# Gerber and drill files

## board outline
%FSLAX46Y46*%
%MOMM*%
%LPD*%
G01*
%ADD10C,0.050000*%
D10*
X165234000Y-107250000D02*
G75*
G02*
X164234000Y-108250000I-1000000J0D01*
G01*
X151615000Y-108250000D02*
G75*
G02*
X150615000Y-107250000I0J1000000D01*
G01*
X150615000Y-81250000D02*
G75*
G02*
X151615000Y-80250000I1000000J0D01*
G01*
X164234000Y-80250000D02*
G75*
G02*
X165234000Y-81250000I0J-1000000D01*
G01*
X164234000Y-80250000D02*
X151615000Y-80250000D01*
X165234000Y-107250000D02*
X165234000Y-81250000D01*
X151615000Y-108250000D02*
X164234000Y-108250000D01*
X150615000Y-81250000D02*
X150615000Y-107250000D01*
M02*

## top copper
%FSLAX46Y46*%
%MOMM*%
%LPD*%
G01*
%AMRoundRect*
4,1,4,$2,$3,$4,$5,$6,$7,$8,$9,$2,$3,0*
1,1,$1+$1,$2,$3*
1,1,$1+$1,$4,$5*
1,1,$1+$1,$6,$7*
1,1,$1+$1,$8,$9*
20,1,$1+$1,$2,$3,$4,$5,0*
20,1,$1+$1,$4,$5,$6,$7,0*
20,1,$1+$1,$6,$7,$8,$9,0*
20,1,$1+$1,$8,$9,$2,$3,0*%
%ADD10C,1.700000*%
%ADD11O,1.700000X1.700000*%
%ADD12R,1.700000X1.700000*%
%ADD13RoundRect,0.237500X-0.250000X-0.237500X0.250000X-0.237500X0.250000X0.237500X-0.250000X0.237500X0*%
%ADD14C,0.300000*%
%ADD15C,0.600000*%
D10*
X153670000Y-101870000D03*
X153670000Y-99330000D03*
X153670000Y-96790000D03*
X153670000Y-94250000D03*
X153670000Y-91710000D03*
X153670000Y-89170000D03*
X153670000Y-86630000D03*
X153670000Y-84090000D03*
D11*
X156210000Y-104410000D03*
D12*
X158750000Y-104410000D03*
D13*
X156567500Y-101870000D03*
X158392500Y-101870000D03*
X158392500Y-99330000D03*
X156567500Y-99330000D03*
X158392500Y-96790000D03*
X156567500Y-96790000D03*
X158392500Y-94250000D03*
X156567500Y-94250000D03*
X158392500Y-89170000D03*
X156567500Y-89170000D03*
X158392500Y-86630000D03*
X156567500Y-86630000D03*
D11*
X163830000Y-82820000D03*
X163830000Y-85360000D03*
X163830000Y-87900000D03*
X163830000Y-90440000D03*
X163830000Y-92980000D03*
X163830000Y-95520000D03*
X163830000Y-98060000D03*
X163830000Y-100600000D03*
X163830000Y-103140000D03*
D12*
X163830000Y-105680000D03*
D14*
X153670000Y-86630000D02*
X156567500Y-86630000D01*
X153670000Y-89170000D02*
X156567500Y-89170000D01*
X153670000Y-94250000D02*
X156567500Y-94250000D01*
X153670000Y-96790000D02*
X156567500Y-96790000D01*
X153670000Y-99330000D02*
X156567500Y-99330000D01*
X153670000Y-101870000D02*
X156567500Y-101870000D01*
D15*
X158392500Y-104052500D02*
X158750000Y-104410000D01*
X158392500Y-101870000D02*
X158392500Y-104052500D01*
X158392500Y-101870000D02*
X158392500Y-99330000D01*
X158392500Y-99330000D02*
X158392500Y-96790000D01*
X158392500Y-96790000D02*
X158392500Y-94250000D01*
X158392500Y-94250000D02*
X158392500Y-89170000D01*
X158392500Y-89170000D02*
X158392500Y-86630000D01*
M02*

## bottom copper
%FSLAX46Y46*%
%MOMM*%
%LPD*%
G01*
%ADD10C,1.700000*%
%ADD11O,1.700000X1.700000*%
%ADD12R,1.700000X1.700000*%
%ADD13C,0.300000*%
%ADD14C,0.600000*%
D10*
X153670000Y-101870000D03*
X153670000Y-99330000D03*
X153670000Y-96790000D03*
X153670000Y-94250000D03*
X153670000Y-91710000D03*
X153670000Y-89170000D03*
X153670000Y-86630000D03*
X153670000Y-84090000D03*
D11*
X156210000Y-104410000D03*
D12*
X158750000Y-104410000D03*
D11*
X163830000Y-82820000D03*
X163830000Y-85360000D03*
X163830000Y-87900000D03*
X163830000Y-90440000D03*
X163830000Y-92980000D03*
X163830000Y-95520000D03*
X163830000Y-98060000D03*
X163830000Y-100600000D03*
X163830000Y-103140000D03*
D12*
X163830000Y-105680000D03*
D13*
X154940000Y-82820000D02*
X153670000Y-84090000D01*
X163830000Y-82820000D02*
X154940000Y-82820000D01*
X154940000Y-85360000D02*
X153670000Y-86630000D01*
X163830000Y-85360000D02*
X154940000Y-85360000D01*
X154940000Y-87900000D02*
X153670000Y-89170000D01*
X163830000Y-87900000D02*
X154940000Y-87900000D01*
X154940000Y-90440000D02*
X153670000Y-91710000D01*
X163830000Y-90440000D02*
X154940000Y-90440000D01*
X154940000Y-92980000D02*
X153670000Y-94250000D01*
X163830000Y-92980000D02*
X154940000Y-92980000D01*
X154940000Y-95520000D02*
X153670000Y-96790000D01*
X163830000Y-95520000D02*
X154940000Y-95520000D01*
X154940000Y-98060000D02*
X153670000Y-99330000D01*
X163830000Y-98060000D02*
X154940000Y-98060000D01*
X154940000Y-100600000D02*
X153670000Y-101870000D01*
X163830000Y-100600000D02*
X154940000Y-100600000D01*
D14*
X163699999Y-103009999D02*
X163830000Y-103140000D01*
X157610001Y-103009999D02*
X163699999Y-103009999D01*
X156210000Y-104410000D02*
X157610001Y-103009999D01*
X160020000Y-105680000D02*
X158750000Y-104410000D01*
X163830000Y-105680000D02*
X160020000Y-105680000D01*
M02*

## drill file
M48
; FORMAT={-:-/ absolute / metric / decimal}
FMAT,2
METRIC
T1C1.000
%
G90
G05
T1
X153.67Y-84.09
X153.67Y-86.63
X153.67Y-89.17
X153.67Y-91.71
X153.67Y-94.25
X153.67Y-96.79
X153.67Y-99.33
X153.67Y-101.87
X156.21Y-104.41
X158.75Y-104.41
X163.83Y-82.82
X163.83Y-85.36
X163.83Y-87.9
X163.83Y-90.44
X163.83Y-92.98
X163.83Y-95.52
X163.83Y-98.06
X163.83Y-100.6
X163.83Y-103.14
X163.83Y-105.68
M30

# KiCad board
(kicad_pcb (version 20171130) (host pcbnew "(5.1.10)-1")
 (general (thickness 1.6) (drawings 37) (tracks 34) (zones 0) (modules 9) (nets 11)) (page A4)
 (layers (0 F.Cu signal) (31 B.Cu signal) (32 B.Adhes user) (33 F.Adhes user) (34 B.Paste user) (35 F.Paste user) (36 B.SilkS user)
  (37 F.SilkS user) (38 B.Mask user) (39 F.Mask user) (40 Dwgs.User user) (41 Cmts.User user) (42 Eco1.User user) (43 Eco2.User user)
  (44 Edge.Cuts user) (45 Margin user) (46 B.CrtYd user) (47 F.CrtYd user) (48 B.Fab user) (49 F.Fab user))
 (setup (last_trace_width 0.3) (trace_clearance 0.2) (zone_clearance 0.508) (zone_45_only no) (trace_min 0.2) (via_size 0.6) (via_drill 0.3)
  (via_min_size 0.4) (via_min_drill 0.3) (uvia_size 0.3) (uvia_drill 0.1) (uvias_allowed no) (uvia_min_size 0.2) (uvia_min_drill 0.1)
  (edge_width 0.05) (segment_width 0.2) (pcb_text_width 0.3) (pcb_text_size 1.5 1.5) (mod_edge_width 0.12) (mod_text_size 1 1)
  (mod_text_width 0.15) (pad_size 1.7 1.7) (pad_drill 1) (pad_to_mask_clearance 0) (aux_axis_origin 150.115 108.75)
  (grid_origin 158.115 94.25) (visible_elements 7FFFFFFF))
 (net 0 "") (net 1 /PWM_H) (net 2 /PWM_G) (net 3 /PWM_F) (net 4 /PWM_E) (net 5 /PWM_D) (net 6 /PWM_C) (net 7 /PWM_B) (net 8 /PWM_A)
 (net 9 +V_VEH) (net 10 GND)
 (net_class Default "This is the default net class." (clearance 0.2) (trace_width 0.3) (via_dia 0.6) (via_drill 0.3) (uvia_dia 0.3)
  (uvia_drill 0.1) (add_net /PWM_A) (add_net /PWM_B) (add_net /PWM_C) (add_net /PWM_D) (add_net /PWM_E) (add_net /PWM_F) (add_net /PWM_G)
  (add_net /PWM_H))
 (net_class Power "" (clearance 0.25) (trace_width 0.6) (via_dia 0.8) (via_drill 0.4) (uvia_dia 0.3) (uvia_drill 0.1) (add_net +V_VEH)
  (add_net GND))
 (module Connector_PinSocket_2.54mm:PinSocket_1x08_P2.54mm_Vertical (layer B.Cu) (at 153.67 84.09 180)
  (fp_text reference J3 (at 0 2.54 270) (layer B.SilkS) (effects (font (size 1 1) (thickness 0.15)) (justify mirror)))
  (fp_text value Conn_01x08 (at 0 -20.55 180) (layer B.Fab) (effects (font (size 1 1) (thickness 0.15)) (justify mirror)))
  (pad 8 thru_hole circle (at 0 -17.78 180) (size 1.7 1.7) (drill 1) (layers *.Cu *.Mask) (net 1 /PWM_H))
  (pad 7 thru_hole circle (at 0 -15.24 180) (size 1.7 1.7) (drill 1) (layers *.Cu *.Mask) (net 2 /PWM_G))
  (pad 6 thru_hole circle (at 0 -12.7 180) (size 1.7 1.7) (drill 1) (layers *.Cu *.Mask) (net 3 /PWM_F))
  (pad 5 thru_hole circle (at 0 -10.16 180) (size 1.7 1.7) (drill 1) (layers *.Cu *.Mask) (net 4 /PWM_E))
  (pad 4 thru_hole circle (at 0 -7.62 180) (size 1.7 1.7) (drill 1) (layers *.Cu *.Mask) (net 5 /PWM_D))
  (pad 3 thru_hole circle (at 0 -5.08 180) (size 1.7 1.7) (drill 1) (layers *.Cu *.Mask) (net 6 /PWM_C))
  (pad 2 thru_hole circle (at 0 -2.54 180) (size 1.7 1.7) (drill 1) (layers *.Cu *.Mask) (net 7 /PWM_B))
  (pad 1 thru_hole circle (at 0 0 180) (size 1.7 1.7) (drill 1) (layers *.Cu *.Mask) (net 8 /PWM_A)))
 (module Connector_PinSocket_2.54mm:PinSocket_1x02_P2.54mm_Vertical (layer B.Cu) (at 158.75 104.41 90)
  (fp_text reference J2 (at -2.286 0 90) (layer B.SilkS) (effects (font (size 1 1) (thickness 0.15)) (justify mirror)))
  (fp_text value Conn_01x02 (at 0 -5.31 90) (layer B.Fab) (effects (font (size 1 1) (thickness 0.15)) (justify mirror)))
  (pad 2 thru_hole oval (at 0 -2.54 90) (size 1.7 1.7) (drill 1) (layers *.Cu *.Mask) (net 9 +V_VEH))
  (pad 1 thru_hole rect (at 0 0 90) (size 1.7 1.7) (drill 1) (layers *.Cu *.Mask) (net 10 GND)))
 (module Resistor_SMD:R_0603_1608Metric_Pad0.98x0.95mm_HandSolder (layer F.Cu) (at 157.48 101.87)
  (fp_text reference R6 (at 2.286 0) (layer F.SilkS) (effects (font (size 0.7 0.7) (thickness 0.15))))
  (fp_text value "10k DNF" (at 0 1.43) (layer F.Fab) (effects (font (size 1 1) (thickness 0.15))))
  (pad 1 smd roundrect (at -0.9125 0) (size 0.975 0.95) (layers F.Cu F.Paste F.Mask) (roundrect_rratio 0.25) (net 1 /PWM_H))
  (pad 2 smd roundrect (at 0.9125 0) (size 0.975 0.95) (layers F.Cu F.Paste F.Mask) (roundrect_rratio 0.25) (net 10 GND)))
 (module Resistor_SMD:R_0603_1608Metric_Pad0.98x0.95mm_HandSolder (layer F.Cu) (at 157.48 99.33)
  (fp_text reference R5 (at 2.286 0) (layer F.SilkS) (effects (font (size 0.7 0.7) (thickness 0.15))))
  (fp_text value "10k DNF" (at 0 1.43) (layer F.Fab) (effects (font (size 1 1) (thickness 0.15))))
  (pad 2 smd roundrect (at 0.9125 0) (size 0.975 0.95) (layers F.Cu F.Paste F.Mask) (roundrect_rratio 0.25) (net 10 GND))
  (pad 1 smd roundrect (at -0.9125 0) (size 0.975 0.95) (layers F.Cu F.Paste F.Mask) (roundrect_rratio 0.25) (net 2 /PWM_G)))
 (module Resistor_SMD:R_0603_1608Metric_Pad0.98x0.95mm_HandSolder (layer F.Cu) (at 157.48 96.79)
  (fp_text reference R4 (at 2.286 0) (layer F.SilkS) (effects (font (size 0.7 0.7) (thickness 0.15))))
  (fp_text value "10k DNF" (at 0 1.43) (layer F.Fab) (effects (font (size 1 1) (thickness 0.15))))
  (pad 2 smd roundrect (at 0.9125 0) (size 0.975 0.95) (layers F.Cu F.Paste F.Mask) (roundrect_rratio 0.25) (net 10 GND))
  (pad 1 smd roundrect (at -0.9125 0) (size 0.975 0.95) (layers F.Cu F.Paste F.Mask) (roundrect_rratio 0.25) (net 3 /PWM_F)))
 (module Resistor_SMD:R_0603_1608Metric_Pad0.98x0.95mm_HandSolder (layer F.Cu) (at 157.48 94.25)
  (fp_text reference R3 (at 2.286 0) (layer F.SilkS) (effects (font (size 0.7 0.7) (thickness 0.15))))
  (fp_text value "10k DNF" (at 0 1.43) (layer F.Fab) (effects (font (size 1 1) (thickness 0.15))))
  (pad 2 smd roundrect (at 0.9125 0) (size 0.975 0.95) (layers F.Cu F.Paste F.Mask) (roundrect_rratio 0.25) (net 10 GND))
  (pad 1 smd roundrect (at -0.9125 0) (size 0.975 0.95) (layers F.Cu F.Paste F.Mask) (roundrect_rratio 0.25) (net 4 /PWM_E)))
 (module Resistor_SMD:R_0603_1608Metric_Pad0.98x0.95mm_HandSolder (layer F.Cu) (at 157.48 89.17)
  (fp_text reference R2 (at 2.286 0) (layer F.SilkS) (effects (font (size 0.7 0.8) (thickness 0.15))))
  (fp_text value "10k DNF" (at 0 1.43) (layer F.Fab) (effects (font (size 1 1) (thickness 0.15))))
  (pad 2 smd roundrect (at 0.9125 0) (size 0.975 0.95) (layers F.Cu F.Paste F.Mask) (roundrect_rratio 0.25) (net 10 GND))
  (pad 1 smd roundrect (at -0.9125 0) (size 0.975 0.95) (layers F.Cu F.Paste F.Mask) (roundrect_rratio 0.25) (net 6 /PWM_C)))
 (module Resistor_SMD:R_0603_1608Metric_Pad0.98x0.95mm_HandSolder (layer F.Cu) (at 157.48 86.63)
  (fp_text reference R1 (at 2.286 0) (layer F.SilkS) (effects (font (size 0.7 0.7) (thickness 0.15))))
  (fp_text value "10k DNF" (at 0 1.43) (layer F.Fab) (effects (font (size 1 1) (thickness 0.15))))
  (pad 2 smd roundrect (at 0.9125 0) (size 0.975 0.95) (layers F.Cu F.Paste F.Mask) (roundrect_rratio 0.25) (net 10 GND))
  (pad 1 smd roundrect (at -0.9125 0) (size 0.975 0.95) (layers F.Cu F.Paste F.Mask) (roundrect_rratio 0.25) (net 7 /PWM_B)))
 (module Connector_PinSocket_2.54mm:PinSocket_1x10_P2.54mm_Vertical (layer B.Cu) (at 163.83 105.68)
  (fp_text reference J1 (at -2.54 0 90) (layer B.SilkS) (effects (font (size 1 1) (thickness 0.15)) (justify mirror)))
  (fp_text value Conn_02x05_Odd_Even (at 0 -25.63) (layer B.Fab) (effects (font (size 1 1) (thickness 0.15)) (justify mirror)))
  (pad 10 thru_hole oval (at 0 -22.86) (size 1.7 1.7) (drill 1) (layers *.Cu *.Mask) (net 8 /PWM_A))
  (pad 9 thru_hole oval (at 0 -20.32) (size 1.7 1.7) (drill 1) (layers *.Cu *.Mask) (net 7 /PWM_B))
  (pad 8 thru_hole oval (at 0 -17.78) (size 1.7 1.7) (drill 1) (layers *.Cu *.Mask) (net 6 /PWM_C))
  (pad 7 thru_hole oval (at 0 -15.24) (size 1.7 1.7) (drill 1) (layers *.Cu *.Mask) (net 5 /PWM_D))
  (pad 6 thru_hole oval (at 0 -12.7) (size 1.7 1.7) (drill 1) (layers *.Cu *.Mask) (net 4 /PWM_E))
  (pad 5 thru_hole oval (at 0 -10.16) (size 1.7 1.7) (drill 1) (layers *.Cu *.Mask) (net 3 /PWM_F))
  (pad 4 thru_hole oval (at 0 -7.62) (size 1.7 1.7) (drill 1) (layers *.Cu *.Mask) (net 2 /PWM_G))
  (pad 3 thru_hole oval (at 0 -5.08) (size 1.7 1.7) (drill 1) (layers *.Cu *.Mask) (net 1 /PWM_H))
  (pad 2 thru_hole oval (at 0 -2.54) (size 1.7 1.7) (drill 1) (layers *.Cu *.Mask) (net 9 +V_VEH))
  (pad 1 thru_hole rect (at 0 0) (size 1.7 1.7) (drill 1) (layers *.Cu *.Mask) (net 10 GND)))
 (gr_arc (start 164.234 107.25) (end 164.234 108.25) (angle -90) (layer Edge.Cuts) (width 0.05))
 (gr_arc (start 151.615 107.25) (end 150.615 107.25) (angle -90) (layer Edge.Cuts) (width 0.05))
 (gr_arc (start 151.615 81.25) (end 151.615 80.25) (angle -90) (layer Edge.Cuts) (width 0.05))
 (gr_arc (start 164.234 81.25) (end 165.234 81.25) (angle -90) (layer Edge.Cuts) (width 0.05))
 (gr_line (start 164.234 80.25) (end 151.615 80.25) (layer Edge.Cuts) (width 0.05))
 (gr_line (start 165.234 107.25) (end 165.234 81.25) (layer Edge.Cuts) (width 0.05))
 (gr_line (start 151.615 108.25) (end 164.234 108.25) (layer Edge.Cuts) (width 0.05))
 (gr_line (start 150.615 81.25) (end 150.615 107.25) (layer Edge.Cuts) (width 0.05))
 (segment (start 154.94 82.82) (end 153.67 84.09) (width 0.3) (layer B.Cu) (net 8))
 (segment (start 163.83 82.82) (end 154.94 82.82) (width 0.3) (layer B.Cu) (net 8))
 (segment (start 153.67 86.63) (end 156.5675 86.63) (width 0.3) (layer F.Cu) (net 7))
 (segment (start 154.94 85.36) (end 153.67 86.63) (width 0.3) (layer B.Cu) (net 7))
 (segment (start 163.83 85.36) (end 154.94 85.36) (width 0.3) (layer B.Cu) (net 7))
 (segment (start 153.67 89.17) (end 156.5675 89.17) (width 0.3) (layer F.Cu) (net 6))
 (segment (start 154.94 87.9) (end 153.67 89.17) (width 0.3) (layer B.Cu) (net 6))
 (segment (start 163.83 87.9) (end 154.94 87.9) (width 0.3) (layer B.Cu) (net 6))
 (segment (start 154.94 90.44) (end 153.67 91.71) (width 0.3) (layer B.Cu) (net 5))
 (segment (start 163.83 90.44) (end 154.94 90.44) (width 0.3) (layer B.Cu) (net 5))
 (segment (start 153.67 94.25) (end 156.5675 94.25) (width 0.3) (layer F.Cu) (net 4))
 (segment (start 154.94 92.98) (end 153.67 94.25) (width 0.3) (layer B.Cu) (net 4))
 (segment (start 163.83 92.98) (end 154.94 92.98) (width 0.3) (layer B.Cu) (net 4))
 (segment (start 153.67 96.79) (end 156.5675 96.79) (width 0.3) (layer F.Cu) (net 3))
 (segment (start 154.94 95.52) (end 153.67 96.79) (width 0.3) (layer B.Cu) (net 3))
 (segment (start 163.83 95.52) (end 154.94 95.52) (width 0.3) (layer B.Cu) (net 3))
 (segment (start 153.67 99.33) (end 156.5675 99.33) (width 0.3) (layer F.Cu) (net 2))
 (segment (start 154.94 98.06) (end 153.67 99.33) (width 0.3) (layer B.Cu) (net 2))
 (segment (start 163.83 98.06) (end 154.94 98.06) (width 0.3) (layer B.Cu) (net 2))
 (segment (start 153.67 101.87) (end 156.5675 101.87) (width 0.3) (layer F.Cu) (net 1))
 (segment (start 154.94 100.6) (end 153.67 101.87) (width 0.3) (layer B.Cu) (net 1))
 (segment (start 163.83 100.6) (end 154.94 100.6) (width 0.3) (layer B.Cu) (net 1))
 (segment (start 163.699999 103.009999) (end 163.83 103.14) (width 0.6) (layer B.Cu) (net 9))
 (segment (start 157.610001 103.009999) (end 163.699999 103.009999) (width 0.6) (layer B.Cu) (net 9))
 (segment (start 156.21 104.41) (end 157.610001 103.009999) (width 0.6) (layer B.Cu) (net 9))
 (segment (start 158.3925 104.0525) (end 158.75 104.41) (width 0.6) (layer F.Cu) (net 10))
 (segment (start 158.3925 101.87) (end 158.3925 104.0525) (width 0.6) (layer F.Cu) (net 10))
 (segment (start 158.3925 101.87) (end 158.3925 99.33) (width 0.6) (layer F.Cu) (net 10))
 (segment (start 158.3925 99.33) (end 158.3925 96.79) (width 0.6) (layer F.Cu) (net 10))
 (segment (start 158.3925 96.79) (end 158.3925 94.25) (width 0.6) (layer F.Cu) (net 10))
 (segment (start 158.3925 94.25) (end 158.3925 89.17) (width 0.6) (layer F.Cu) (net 10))
 (segment (start 158.3925 89.17) (end 158.3925 86.63) (width 0.6) (layer F.Cu) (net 10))
 (segment (start 160.02 105.68) (end 158.75 104.41) (width 0.6) (layer B.Cu) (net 10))
 (segment (start 163.83 105.68) (end 160.02 105.68) (width 0.6) (layer B.Cu) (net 10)))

